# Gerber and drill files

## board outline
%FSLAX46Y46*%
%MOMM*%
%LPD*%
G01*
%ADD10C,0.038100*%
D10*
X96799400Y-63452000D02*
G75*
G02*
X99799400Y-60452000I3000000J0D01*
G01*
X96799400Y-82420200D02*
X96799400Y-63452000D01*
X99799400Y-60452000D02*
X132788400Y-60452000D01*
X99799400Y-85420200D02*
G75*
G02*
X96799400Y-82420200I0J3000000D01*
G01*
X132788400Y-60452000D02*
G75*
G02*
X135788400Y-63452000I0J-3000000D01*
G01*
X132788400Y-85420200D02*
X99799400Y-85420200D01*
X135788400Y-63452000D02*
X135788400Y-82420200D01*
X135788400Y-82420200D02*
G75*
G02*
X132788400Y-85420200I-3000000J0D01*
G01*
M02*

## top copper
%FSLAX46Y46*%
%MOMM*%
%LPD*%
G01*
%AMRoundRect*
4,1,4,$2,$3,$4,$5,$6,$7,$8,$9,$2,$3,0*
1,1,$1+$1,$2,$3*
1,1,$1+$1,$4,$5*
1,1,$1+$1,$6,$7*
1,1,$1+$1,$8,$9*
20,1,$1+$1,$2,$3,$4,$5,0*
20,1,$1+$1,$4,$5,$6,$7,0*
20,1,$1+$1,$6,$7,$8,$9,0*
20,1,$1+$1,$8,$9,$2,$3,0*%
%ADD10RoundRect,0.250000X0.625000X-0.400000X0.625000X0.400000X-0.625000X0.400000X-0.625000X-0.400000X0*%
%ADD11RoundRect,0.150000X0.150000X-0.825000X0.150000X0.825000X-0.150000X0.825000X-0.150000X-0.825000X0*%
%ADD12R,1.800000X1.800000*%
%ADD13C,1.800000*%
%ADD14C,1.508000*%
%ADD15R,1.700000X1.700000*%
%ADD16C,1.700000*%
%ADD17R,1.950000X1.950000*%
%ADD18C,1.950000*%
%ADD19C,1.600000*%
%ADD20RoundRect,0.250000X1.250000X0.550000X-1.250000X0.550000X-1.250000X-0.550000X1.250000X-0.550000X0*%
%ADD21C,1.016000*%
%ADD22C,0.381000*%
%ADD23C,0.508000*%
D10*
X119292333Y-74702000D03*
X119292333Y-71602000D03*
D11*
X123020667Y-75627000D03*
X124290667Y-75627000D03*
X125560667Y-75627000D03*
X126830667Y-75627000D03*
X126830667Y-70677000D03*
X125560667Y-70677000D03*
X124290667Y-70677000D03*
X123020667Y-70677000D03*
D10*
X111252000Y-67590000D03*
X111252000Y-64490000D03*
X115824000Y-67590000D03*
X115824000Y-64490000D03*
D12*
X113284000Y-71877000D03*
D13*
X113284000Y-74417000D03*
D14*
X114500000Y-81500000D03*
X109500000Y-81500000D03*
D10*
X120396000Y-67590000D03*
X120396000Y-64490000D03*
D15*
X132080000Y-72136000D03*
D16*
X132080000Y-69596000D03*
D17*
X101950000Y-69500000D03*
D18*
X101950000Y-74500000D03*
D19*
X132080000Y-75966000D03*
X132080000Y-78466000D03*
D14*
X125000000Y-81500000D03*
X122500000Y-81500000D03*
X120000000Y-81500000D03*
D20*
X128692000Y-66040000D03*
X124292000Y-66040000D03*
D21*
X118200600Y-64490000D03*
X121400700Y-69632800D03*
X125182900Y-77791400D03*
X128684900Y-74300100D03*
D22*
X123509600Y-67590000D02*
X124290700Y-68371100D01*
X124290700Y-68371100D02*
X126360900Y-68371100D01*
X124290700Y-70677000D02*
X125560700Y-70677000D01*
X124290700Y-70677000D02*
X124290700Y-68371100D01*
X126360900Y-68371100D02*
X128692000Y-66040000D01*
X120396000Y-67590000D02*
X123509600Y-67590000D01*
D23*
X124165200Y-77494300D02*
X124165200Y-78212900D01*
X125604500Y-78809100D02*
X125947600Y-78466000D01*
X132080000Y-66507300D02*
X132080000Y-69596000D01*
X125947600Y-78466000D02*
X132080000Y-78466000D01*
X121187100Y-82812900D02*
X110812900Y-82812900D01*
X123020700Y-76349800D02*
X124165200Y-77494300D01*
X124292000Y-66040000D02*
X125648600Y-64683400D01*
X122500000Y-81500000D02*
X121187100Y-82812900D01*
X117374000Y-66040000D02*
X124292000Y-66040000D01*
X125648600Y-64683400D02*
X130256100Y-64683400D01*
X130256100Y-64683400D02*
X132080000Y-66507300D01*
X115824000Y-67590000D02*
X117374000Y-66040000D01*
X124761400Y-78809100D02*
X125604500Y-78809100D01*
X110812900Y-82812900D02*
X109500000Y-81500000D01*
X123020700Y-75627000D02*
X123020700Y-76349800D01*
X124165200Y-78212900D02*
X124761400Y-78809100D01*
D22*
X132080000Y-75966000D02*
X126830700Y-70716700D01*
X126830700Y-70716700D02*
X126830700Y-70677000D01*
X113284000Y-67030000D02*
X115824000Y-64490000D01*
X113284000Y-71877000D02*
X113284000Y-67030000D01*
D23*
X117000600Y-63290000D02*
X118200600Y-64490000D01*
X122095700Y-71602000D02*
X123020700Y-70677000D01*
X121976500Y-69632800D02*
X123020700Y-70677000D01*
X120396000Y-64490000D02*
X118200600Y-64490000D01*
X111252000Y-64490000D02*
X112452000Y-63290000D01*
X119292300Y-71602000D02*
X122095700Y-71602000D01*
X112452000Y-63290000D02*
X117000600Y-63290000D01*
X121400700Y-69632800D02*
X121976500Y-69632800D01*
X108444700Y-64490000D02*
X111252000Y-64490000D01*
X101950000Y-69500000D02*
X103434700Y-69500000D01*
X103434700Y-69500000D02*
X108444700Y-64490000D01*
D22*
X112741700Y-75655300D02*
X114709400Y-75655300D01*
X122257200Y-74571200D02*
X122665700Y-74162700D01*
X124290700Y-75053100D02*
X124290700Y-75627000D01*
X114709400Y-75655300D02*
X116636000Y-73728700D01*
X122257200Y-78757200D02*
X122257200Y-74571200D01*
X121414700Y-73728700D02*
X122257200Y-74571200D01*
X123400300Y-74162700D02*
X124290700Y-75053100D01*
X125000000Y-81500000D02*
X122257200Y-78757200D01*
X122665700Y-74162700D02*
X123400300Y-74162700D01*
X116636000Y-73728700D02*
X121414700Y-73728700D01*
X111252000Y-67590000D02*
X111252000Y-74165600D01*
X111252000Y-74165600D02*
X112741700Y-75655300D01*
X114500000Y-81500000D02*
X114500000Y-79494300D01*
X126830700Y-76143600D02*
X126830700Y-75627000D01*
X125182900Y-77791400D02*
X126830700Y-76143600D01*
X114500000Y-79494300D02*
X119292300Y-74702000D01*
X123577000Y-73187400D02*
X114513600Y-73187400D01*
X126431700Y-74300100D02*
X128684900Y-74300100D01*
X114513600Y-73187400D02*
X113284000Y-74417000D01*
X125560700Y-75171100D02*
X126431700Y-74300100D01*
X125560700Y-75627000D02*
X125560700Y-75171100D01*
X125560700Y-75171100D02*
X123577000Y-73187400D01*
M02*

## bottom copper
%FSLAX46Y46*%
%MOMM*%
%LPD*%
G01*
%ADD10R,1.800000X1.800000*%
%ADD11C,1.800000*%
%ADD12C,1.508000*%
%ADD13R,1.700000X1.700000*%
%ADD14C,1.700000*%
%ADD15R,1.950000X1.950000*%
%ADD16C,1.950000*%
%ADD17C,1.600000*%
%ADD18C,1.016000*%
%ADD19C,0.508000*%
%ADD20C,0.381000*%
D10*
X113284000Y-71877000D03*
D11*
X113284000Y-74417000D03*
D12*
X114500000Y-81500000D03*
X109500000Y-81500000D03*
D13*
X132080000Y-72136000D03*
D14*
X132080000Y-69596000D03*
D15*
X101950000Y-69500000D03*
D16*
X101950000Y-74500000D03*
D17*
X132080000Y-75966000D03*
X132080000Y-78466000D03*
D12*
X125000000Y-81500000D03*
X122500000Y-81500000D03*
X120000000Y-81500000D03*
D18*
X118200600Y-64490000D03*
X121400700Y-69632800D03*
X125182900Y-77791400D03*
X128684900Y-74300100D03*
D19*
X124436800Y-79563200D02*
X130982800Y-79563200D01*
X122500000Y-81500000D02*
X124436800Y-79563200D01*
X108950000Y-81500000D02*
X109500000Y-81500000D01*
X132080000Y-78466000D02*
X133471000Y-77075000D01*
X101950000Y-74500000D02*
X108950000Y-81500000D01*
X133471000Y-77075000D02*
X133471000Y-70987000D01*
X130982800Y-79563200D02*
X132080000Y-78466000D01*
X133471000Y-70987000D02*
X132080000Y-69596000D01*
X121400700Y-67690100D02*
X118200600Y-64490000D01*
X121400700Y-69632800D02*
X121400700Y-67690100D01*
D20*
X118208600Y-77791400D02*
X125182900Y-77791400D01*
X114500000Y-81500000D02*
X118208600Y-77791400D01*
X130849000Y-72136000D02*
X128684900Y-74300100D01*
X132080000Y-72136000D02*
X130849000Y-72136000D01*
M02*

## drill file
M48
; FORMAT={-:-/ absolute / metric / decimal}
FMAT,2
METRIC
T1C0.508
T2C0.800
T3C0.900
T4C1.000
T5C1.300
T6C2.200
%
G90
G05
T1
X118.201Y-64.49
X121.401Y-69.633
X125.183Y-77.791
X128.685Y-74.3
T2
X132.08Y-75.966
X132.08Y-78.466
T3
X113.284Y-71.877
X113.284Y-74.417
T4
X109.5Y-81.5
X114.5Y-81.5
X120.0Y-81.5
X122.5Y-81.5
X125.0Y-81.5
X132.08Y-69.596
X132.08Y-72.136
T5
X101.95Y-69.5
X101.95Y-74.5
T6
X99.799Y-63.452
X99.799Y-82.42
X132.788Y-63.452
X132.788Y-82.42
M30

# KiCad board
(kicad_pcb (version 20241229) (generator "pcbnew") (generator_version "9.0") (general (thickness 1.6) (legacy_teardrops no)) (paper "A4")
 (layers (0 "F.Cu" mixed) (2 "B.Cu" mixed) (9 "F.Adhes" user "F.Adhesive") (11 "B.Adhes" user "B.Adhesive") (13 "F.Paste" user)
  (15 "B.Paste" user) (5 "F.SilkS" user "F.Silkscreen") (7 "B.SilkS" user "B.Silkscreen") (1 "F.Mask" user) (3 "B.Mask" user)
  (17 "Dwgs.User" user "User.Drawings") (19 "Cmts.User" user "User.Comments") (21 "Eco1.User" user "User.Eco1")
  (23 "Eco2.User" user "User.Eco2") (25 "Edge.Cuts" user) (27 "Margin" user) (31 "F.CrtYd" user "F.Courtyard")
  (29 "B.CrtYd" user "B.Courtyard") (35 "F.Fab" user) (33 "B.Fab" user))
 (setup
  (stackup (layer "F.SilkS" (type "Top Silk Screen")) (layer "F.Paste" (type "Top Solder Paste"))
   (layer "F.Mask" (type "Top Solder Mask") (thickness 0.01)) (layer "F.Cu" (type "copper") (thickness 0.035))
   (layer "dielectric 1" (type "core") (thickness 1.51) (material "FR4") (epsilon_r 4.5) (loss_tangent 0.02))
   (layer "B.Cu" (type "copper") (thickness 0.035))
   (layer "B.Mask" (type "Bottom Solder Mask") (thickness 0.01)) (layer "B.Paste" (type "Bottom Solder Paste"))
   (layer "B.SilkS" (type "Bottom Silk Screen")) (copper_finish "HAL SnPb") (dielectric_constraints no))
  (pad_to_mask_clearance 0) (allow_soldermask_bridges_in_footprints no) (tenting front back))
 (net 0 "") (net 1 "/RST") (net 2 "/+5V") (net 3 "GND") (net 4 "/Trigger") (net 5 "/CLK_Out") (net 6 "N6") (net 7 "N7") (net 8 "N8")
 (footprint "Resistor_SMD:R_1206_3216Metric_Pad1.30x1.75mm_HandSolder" (layer "F.Cu") (at 119.292333 73.152 90)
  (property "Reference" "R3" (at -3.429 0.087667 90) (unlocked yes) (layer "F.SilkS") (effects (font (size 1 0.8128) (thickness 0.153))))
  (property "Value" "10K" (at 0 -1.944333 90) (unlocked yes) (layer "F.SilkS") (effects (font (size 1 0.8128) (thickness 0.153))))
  (pad "1" smd roundrect (at -1.55 0 90) (size 1.3 1.75) (layers "F.Cu" "F.Mask" "F.Paste") (roundrect_rratio 0.192308) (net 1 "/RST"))
  (pad "2" smd roundrect (at 1.55 0 90) (size 1.3 1.75) (layers "F.Cu" "F.Mask" "F.Paste") (roundrect_rratio 0.192308) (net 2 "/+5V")))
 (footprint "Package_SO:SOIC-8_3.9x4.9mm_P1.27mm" (layer "F.Cu") (at 124.925667 73.152 90)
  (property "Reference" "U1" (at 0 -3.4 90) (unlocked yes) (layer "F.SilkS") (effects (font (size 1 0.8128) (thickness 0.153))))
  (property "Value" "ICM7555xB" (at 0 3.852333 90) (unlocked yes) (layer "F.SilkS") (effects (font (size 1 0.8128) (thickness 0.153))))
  (pad "1" smd roundrect (at -2.475 -1.905 90) (size 1.95 0.6) (layers "F.Cu" "F.Mask" "F.Paste") (roundrect_rratio 0.25) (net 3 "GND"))
  (pad "2" smd roundrect (at -2.475 -0.635 90) (size 1.95 0.6) (layers "F.Cu" "F.Mask" "F.Paste") (roundrect_rratio 0.25) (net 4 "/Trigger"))
  (pad "3" smd roundrect (at -2.475 0.635 90) (size 1.95 0.6) (layers "F.Cu" "F.Mask" "F.Paste") (roundrect_rratio 0.25) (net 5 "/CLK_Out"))
  (pad "4" smd roundrect (at -2.475 1.905 90) (size 1.95 0.6) (layers "F.Cu" "F.Mask" "F.Paste") (roundrect_rratio 0.25) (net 1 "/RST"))
  (pad "5" smd roundrect (at 2.475 1.905 90) (size 1.95 0.6) (layers "F.Cu" "F.Mask" "F.Paste") (roundrect_rratio 0.25) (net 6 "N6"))
  (pad "6" smd roundrect (at 2.475 0.635 90) (size 1.95 0.6) (layers "F.Cu" "F.Mask" "F.Paste") (roundrect_rratio 0.25) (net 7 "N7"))
  (pad "7" smd roundrect (at 2.475 -0.635 90) (size 1.95 0.6) (layers "F.Cu" "F.Mask" "F.Paste") (roundrect_rratio 0.25) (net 7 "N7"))
  (pad "8" smd roundrect (at 2.475 -1.905 90) (size 1.95 0.6) (layers "F.Cu" "F.Mask" "F.Paste") (roundrect_rratio 0.25) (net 2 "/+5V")))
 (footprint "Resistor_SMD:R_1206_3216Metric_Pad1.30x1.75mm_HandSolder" (layer "F.Cu") (at 111.252 66.04 90)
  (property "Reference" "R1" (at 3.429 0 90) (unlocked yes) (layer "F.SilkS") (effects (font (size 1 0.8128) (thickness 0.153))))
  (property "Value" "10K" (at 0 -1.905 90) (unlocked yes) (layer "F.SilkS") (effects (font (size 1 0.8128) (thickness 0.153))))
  (pad "1" smd roundrect (at -1.55 0 90) (size 1.3 1.75) (layers "F.Cu" "F.Mask" "F.Paste") (roundrect_rratio 0.192308) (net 4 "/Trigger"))
  (pad "2" smd roundrect (at 1.55 0 90) (size 1.3 1.75) (layers "F.Cu" "F.Mask" "F.Paste") (roundrect_rratio 0.192308) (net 2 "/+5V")))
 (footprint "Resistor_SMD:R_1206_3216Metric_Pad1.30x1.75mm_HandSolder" (layer "F.Cu") (at 115.824 66.04 90)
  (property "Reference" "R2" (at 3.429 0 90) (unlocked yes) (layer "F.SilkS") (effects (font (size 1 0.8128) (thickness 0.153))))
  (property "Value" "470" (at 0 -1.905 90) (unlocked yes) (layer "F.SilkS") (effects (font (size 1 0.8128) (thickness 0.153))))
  (pad "1" smd roundrect (at -1.55 0 90) (size 1.3 1.75) (layers "F.Cu" "F.Mask" "F.Paste") (roundrect_rratio 0.192308) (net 3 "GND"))
  (pad "2" smd roundrect (at 1.55 0 90) (size 1.3 1.75) (layers "F.Cu" "F.Mask" "F.Paste") (roundrect_rratio 0.192308) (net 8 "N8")))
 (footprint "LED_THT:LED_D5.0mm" (layer "F.Cu") (at 113.284 71.877 -90)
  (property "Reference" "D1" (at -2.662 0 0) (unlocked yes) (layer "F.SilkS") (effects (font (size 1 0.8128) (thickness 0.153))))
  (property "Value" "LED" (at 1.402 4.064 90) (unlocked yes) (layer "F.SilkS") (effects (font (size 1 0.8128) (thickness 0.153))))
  (pad "1" thru_hole rect (at 0 0 270) (size 1.8 1.8) (drill 0.9) (layers "*.Cu" "*.Mask") (remove_unused_layers no) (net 8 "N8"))
  (pad "2" thru_hole circle (at 2.54 0 270) (size 1.8 1.8) (drill 0.9) (layers "*.Cu" "*.Mask") (remove_unused_layers no) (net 5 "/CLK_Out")))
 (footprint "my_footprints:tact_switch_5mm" (layer "F.Cu") (at 112 81.5 180)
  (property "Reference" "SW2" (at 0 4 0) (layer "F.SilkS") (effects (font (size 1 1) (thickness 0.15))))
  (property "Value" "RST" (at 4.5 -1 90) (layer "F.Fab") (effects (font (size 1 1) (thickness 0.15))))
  (pad "1" thru_hole circle (at -2.5 0 180) (size 1.508 1.508) (drill 1) (layers "*.Cu" "*.Mask") (remove_unused_layers no) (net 1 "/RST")
   (solder_mask_margin 0.102))
  (pad "2" thru_hole circle (at 2.5 0 180) (size 1.508 1.508) (drill 1) (layers "*.Cu" "*.Mask") (remove_unused_layers no) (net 3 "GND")
   (solder_mask_margin 0.102)))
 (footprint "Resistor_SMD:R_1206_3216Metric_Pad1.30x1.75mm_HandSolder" (layer "F.Cu") (at 120.396 66.04 90)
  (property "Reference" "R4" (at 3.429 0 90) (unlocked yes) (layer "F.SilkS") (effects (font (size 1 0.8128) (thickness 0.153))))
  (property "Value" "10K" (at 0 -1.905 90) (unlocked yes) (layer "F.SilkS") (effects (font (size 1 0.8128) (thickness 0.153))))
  (pad "1" smd roundrect (at -1.55 0 90) (size 1.3 1.75) (layers "F.Cu" "F.Mask" "F.Paste") (roundrect_rratio 0.192308) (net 7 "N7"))
  (pad "2" smd roundrect (at 1.55 0 90) (size 1.3 1.75) (layers "F.Cu" "F.Mask" "F.Paste") (roundrect_rratio 0.192308) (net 2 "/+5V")))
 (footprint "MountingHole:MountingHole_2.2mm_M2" (layer "F.Cu") (at 99.7994 63.452)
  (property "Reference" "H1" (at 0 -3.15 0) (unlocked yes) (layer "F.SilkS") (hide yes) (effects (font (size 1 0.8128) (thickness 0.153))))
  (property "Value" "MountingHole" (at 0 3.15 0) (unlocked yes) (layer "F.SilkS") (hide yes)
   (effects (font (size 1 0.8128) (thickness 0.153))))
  (pad "" np_thru_hole circle (at 0 0) (size 2.2 2.2) (drill 2.2) (layers "*.Cu" "*.Mask")))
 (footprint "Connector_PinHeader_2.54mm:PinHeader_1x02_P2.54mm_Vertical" (layer "F.Cu") (at 132.08 72.136 180)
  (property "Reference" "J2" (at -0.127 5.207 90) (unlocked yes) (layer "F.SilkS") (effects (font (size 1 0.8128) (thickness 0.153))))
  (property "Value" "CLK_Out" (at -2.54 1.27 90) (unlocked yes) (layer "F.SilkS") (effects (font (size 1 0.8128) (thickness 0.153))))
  (pad "1" thru_hole rect (at 0 0 180) (size 1.7 1.7) (drill 1) (layers "*.Cu" "*.Mask") (remove_unused_layers no) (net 5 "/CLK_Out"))
  (pad "2" thru_hole circle (at 0 2.54 180) (size 1.7 1.7) (drill 1) (layers "*.Cu" "*.Mask") (remove_unused_layers no) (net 3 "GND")))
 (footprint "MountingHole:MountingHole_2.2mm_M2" (layer "F.Cu") (at 132.7884 82.4202)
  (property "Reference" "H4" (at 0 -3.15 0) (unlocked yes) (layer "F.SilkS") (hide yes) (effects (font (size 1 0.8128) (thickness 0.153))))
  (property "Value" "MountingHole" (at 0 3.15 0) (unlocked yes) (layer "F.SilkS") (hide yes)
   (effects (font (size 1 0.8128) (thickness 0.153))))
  (pad "" np_thru_hole circle (at 0 0) (size 2.2 2.2) (drill 2.2) (layers "*.Cu" "*.Mask")))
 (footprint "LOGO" (layer "F.Cu") (at 105.5 63.5)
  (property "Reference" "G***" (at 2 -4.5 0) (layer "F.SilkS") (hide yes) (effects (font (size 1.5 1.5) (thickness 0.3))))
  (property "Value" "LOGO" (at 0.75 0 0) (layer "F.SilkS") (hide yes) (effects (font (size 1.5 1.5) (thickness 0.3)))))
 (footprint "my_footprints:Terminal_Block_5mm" (layer "F.Cu") (at 101.95 72 -90)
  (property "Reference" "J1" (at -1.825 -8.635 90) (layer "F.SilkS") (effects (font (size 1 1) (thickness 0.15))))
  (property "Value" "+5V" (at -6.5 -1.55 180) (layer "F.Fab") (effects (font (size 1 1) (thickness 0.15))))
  (pad "1" thru_hole rect (at -2.5 0 270) (size 1.95 1.95) (drill 1.3) (layers "*.Cu" "*.Mask") (remove_unused_layers no) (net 2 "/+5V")
   (solder_mask_margin 0.102))
  (pad "2" thru_hole circle (at 2.5 0 270) (size 1.95 1.95) (drill 1.3) (layers "*.Cu" "*.Mask") (remove_unused_layers no) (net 3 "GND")
   (solder_mask_margin 0.102)))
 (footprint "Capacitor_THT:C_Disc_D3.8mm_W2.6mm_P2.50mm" (layer "F.Cu") (at 132.08 75.966 -90)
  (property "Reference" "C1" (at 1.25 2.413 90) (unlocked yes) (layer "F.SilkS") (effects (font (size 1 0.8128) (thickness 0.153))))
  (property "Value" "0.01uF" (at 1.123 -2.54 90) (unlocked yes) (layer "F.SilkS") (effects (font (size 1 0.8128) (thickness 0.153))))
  (pad "1" thru_hole circle (at 0 0 270) (size 1.6 1.6) (drill 0.8) (layers "*.Cu" "*.Mask") (remove_unused_layers no) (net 6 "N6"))
  (pad "2" thru_hole circle (at 2.5 0 270) (size 1.6 1.6) (drill 0.8) (layers "*.Cu" "*.Mask") (remove_unused_layers no) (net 3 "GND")))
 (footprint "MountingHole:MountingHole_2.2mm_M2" (layer "F.Cu") (at 132.7884 63.452)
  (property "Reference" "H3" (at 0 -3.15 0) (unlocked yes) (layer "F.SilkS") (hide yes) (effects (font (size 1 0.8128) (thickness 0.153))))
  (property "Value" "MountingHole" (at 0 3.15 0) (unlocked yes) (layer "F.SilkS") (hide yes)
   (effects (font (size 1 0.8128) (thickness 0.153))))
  (pad "" np_thru_hole circle (at 0 0) (size 2.2 2.2) (drill 2.2) (layers "*.Cu" "*.Mask")))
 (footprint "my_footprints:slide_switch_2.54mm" (layer "F.Cu") (at 122.5 81.5 180)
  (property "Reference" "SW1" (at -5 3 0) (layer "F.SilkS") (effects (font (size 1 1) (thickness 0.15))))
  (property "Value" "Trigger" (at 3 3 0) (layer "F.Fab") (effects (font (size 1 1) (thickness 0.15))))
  (pad "1" thru_hole circle (at -2.5 0 180) (size 1.508 1.508) (drill 1) (layers "*.Cu" "*.Mask") (remove_unused_layers no)
   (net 4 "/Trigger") (solder_mask_margin 0.102))
  (pad "2" thru_hole circle (at 0 0 180) (size 1.508 1.508) (drill 1) (layers "*.Cu" "*.Mask") (remove_unused_layers no) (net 3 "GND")
   (solder_mask_margin 0.102))
  (pad "3" thru_hole circle (at 2.5 0 180) (size 1.508 1.508) (drill 1) (layers "*.Cu" "*.Mask") (remove_unused_layers no)
   (solder_mask_margin 0.102)))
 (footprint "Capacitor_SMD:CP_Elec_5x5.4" (layer "F.Cu") (at 126.492 66.04 180)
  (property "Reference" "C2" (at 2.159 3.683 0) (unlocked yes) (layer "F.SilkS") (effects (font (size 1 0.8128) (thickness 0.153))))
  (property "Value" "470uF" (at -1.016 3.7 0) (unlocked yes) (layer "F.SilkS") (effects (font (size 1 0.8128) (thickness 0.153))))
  (pad "1" smd roundrect (at -2.2 0 180) (size 3 1.6) (layers "F.Cu" "F.Mask" "F.Paste") (roundrect_rratio 0.15625) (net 7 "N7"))
  (pad "2" smd roundrect (at 2.2 0 180) (size 3 1.6) (layers "F.Cu" "F.Mask" "F.Paste") (roundrect_rratio 0.15625) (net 3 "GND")))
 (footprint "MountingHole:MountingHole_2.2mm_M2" (layer "F.Cu") (at 99.7994 82.4202)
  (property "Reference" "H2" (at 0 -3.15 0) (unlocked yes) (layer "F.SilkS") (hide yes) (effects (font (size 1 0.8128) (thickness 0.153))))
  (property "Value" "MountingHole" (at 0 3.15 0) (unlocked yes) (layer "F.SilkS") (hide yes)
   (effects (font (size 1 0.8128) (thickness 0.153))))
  (pad "" np_thru_hole circle (at 0 0) (size 2.2 2.2) (drill 2.2) (layers "*.Cu" "*.Mask")))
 (gr_arc (start 96.7994 63.452) (mid 97.67808 61.33068) (end 99.7994 60.452) (stroke (width 0.0381) (type default)) (layer "Edge.Cuts"))
 (gr_line (start 96.7994 82.4202) (end 96.7994 63.452) (stroke (width 0.0381) (type default)) (layer "Edge.Cuts"))
 (gr_line (start 99.7994 60.452) (end 132.7884 60.452) (stroke (width 0.0381) (type default)) (layer "Edge.Cuts"))
 (gr_arc (start 99.7994 85.4202) (mid 97.67808 84.54152) (end 96.7994 82.4202) (stroke (width 0.0381) (type default)) (layer "Edge.Cuts"))
 (gr_arc (start 132.7884 60.452) (mid 134.90972 61.33068) (end 135.7884 63.452) (stroke (width 0.0381) (type default)) (layer "Edge.Cuts"))
 (gr_line (start 132.7884 85.4202) (end 99.7994 85.4202) (stroke (width 0.0381) (type default)) (layer "Edge.Cuts"))
 (gr_line (start 135.7884 63.452) (end 135.7884 82.4202) (stroke (width 0.0381) (type default)) (layer "Edge.Cuts"))
 (gr_arc (start 135.7884 82.4202) (mid 134.90972 84.54152) (end 132.7884 85.4202) (stroke (width 0.0381) (type default)) (layer "Edge.Cuts"))
 (segment (start 123.509600 67.590000) (end 124.290700 68.371100) (width 0.381000) (layer "F.Cu") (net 7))
 (segment (start 124.290700 68.371100) (end 126.360900 68.371100) (width 0.381000) (layer "F.Cu") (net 7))
 (segment (start 124.290700 70.677000) (end 125.560700 70.677000) (width 0.381000) (layer "F.Cu") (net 7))
 (segment (start 124.290700 70.677000) (end 124.290700 68.371100) (width 0.381000) (layer "F.Cu") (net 7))
 (segment (start 126.360900 68.371100) (end 128.692000 66.040000) (width 0.381000) (layer "F.Cu") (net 7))
 (segment (start 120.396000 67.590000) (end 123.509600 67.590000) (width 0.381000) (layer "F.Cu") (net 7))
 (segment (start 124.165200 77.494300) (end 124.165200 78.212900) (width 0.508000) (layer "F.Cu") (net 3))
 (segment (start 125.604500 78.809100) (end 125.947600 78.466000) (width 0.508000) (layer "F.Cu") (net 3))
 (segment (start 132.080000 66.507300) (end 132.080000 69.596000) (width 0.508000) (layer "F.Cu") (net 3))
 (segment (start 125.947600 78.466000) (end 132.080000 78.466000) (width 0.508000) (layer "F.Cu") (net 3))
 (segment (start 121.187100 82.812900) (end 110.812900 82.812900) (width 0.508000) (layer "F.Cu") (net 3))
 (segment (start 123.020700 76.349800) (end 124.165200 77.494300) (width 0.508000) (layer "F.Cu") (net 3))
 (segment (start 124.292000 66.040000) (end 125.648600 64.683400) (width 0.508000) (layer "F.Cu") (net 3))
 (segment (start 122.500000 81.500000) (end 121.187100 82.812900) (width 0.508000) (layer "F.Cu") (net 3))
 (segment (start 117.374000 66.040000) (end 124.292000 66.040000) (width 0.508000) (layer "F.Cu") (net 3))
 (segment (start 125.648600 64.683400) (end 130.256100 64.683400) (width 0.508000) (layer "F.Cu") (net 3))
 (segment (start 130.256100 64.683400) (end 132.080000 66.507300) (width 0.508000) (layer "F.Cu") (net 3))
 (segment (start 115.824000 67.590000) (end 117.374000 66.040000) (width 0.508000) (layer "F.Cu") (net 3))
 (segment (start 124.761400 78.809100) (end 125.604500 78.809100) (width 0.508000) (layer "F.Cu") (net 3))
 (segment (start 110.812900 82.812900) (end 109.500000 81.500000) (width 0.508000) (layer "F.Cu") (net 3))
 (segment (start 123.020700 75.627000) (end 123.020700 76.349800) (width 0.508000) (layer "F.Cu") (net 3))
 (segment (start 124.165200 78.212900) (end 124.761400 78.809100) (width 0.508000) (layer "F.Cu") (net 3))
 (segment (start 124.436800 79.563200) (end 130.982800 79.563200) (width 0.508000) (layer "B.Cu") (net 3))
 (segment (start 122.500000 81.500000) (end 124.436800 79.563200) (width 0.508000) (layer "B.Cu") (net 3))
 (segment (start 108.950000 81.500000) (end 109.500000 81.500000) (width 0.508000) (layer "B.Cu") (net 3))
 (segment (start 132.080000 78.466000) (end 133.471000 77.075000) (width 0.508000) (layer "B.Cu") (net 3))
 (segment (start 101.950000 74.500000) (end 108.950000 81.500000) (width 0.508000) (layer "B.Cu") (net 3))
 (segment (start 133.471000 77.075000) (end 133.471000 70.987000) (width 0.508000) (layer "B.Cu") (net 3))
 (segment (start 130.982800 79.563200) (end 132.080000 78.466000) (width 0.508000) (layer "B.Cu") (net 3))
 (segment (start 133.471000 70.987000) (end 132.080000 69.596000) (width 0.508000) (layer "B.Cu") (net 3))
 (segment (start 132.080000 75.966000) (end 126.830700 70.716700) (width 0.381000) (layer "F.Cu") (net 6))
 (segment (start 126.830700 70.716700) (end 126.830700 70.677000) (width 0.381000) (layer "F.Cu") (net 6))
 (segment (start 113.284000 67.030000) (end 115.824000 64.490000) (width 0.381000) (layer "F.Cu") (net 8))
 (segment (start 113.284000 71.877000) (end 113.284000 67.030000) (width 0.381000) (layer "F.Cu") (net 8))
 (segment (start 117.000600 63.290000) (end 118.200600 64.490000) (width 0.508000) (layer "F.Cu") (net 2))
 (segment (start 122.095700 71.602000) (end 123.020700 70.677000) (width 0.508000) (layer "F.Cu") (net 2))
 (segment (start 121.976500 69.632800) (end 123.020700 70.677000) (width 0.508000) (layer "F.Cu") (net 2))
 (segment (start 120.396000 64.490000) (end 118.200600 64.490000) (width 0.508000) (layer "F.Cu") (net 2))
 (segment (start 111.252000 64.490000) (end 112.452000 63.290000) (width 0.508000) (layer "F.Cu") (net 2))
 (segment (start 119.292300 71.602000) (end 122.095700 71.602000) (width 0.508000) (layer "F.Cu") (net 2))
 (segment (start 112.452000 63.290000) (end 117.000600 63.290000) (width 0.508000) (layer "F.Cu") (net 2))
 (segment (start 121.400700 69.632800) (end 121.976500 69.632800) (width 0.508000) (layer "F.Cu") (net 2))
 (segment (start 108.444700 64.490000) (end 111.252000 64.490000) (width 0.508000) (layer "F.Cu") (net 2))
 (segment (start 101.950000 69.500000) (end 103.434700 69.500000) (width 0.508000) (layer "F.Cu") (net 2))
 (segment (start 103.434700 69.500000) (end 108.444700 64.490000) (width 0.508000) (layer "F.Cu") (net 2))
 (segment (start 121.400700 67.690100) (end 118.200600 64.490000) (width 0.508000) (layer "B.Cu") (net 2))
 (segment (start 121.400700 69.632800) (end 121.400700 67.690100) (width 0.508000) (layer "B.Cu") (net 2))
 (segment (start 112.741700 75.655300) (end 114.709400 75.655300) (width 0.381000) (layer "F.Cu") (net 4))
 (segment (start 122.257200 74.571200) (end 122.665700 74.162700) (width 0.381000) (layer "F.Cu") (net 4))
 (segment (start 124.290700 75.053100) (end 124.290700 75.627000) (width 0.381000) (layer "F.Cu") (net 4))
 (segment (start 114.709400 75.655300) (end 116.636000 73.728700) (width 0.381000) (layer "F.Cu") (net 4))
 (segment (start 122.257200 78.757200) (end 122.257200 74.571200) (width 0.381000) (layer "F.Cu") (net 4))
 (segment (start 121.414700 73.728700) (end 122.257200 74.571200) (width 0.381000) (layer "F.Cu") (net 4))
 (segment (start 123.400300 74.162700) (end 124.290700 75.053100) (width 0.381000) (layer "F.Cu") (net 4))
 (segment (start 125.000000 81.500000) (end 122.257200 78.757200) (width 0.381000) (layer "F.Cu") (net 4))
 (segment (start 122.665700 74.162700) (end 123.400300 74.162700) (width 0.381000) (layer "F.Cu") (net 4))
 (segment (start 116.636000 73.728700) (end 121.414700 73.728700) (width 0.381000) (layer "F.Cu") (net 4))
 (segment (start 111.252000 67.590000) (end 111.252000 74.165600) (width 0.381000) (layer "F.Cu") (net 4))
 (segment (start 111.252000 74.165600) (end 112.741700 75.655300) (width 0.381000) (layer "F.Cu") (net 4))
 (segment (start 114.500000 81.500000) (end 114.500000 79.494300) (width 0.381000) (layer "F.Cu") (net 1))
 (segment (start 126.830700 76.143600) (end 126.830700 75.627000) (width 0.381000) (layer "F.Cu") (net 1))
 (segment (start 125.182900 77.791400) (end 126.830700 76.143600) (width 0.381000) (layer "F.Cu") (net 1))
 (segment (start 114.500000 79.494300) (end 119.292300 74.702000) (width 0.381000) (layer "F.Cu") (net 1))
 (segment (start 118.208600 77.791400) (end 125.182900 77.791400) (width 0.381000) (layer "B.Cu") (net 1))
 (segment (start 114.500000 81.500000) (end 118.208600 77.791400) (width 0.381000) (layer "B.Cu") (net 1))
 (segment (start 123.577000 73.187400) (end 114.513600 73.187400) (width 0.381000) (layer "F.Cu") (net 5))
 (segment (start 126.431700 74.300100) (end 128.684900 74.300100) (width 0.381000) (layer "F.Cu") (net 5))
 (segment (start 114.513600 73.187400) (end 113.284000 74.417000) (width 0.381000) (layer "F.Cu") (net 5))
 (segment (start 125.560700 75.171100) (end 126.431700 74.300100) (width 0.381000) (layer "F.Cu") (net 5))
 (segment (start 125.560700 75.627000) (end 125.560700 75.171100) (width 0.381000) (layer "F.Cu") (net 5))
 (segment (start 125.560700 75.171100) (end 123.577000 73.187400) (width 0.381000) (layer "F.Cu") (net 5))
 (segment (start 130.849000 72.136000) (end 128.684900 74.300100) (width 0.381000) (layer "B.Cu") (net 5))
 (segment (start 132.080000 72.136000) (end 130.849000 72.136000) (width 0.381000) (layer "B.Cu") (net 5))
 (via (at 118.200600 64.490000) (size 1.016000) (drill 0.508000) (layers "F.Cu" "B.Cu") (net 2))
 (via (at 121.400700 69.632800) (size 1.016000) (drill 0.508000) (layers "F.Cu" "B.Cu") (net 2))
 (via (at 125.182900 77.791400) (size 1.016000) (drill 0.508000) (layers "F.Cu" "B.Cu") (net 1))
 (via (at 128.684900 74.300100) (size 1.016000) (drill 0.508000) (layers "F.Cu" "B.Cu") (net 5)))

